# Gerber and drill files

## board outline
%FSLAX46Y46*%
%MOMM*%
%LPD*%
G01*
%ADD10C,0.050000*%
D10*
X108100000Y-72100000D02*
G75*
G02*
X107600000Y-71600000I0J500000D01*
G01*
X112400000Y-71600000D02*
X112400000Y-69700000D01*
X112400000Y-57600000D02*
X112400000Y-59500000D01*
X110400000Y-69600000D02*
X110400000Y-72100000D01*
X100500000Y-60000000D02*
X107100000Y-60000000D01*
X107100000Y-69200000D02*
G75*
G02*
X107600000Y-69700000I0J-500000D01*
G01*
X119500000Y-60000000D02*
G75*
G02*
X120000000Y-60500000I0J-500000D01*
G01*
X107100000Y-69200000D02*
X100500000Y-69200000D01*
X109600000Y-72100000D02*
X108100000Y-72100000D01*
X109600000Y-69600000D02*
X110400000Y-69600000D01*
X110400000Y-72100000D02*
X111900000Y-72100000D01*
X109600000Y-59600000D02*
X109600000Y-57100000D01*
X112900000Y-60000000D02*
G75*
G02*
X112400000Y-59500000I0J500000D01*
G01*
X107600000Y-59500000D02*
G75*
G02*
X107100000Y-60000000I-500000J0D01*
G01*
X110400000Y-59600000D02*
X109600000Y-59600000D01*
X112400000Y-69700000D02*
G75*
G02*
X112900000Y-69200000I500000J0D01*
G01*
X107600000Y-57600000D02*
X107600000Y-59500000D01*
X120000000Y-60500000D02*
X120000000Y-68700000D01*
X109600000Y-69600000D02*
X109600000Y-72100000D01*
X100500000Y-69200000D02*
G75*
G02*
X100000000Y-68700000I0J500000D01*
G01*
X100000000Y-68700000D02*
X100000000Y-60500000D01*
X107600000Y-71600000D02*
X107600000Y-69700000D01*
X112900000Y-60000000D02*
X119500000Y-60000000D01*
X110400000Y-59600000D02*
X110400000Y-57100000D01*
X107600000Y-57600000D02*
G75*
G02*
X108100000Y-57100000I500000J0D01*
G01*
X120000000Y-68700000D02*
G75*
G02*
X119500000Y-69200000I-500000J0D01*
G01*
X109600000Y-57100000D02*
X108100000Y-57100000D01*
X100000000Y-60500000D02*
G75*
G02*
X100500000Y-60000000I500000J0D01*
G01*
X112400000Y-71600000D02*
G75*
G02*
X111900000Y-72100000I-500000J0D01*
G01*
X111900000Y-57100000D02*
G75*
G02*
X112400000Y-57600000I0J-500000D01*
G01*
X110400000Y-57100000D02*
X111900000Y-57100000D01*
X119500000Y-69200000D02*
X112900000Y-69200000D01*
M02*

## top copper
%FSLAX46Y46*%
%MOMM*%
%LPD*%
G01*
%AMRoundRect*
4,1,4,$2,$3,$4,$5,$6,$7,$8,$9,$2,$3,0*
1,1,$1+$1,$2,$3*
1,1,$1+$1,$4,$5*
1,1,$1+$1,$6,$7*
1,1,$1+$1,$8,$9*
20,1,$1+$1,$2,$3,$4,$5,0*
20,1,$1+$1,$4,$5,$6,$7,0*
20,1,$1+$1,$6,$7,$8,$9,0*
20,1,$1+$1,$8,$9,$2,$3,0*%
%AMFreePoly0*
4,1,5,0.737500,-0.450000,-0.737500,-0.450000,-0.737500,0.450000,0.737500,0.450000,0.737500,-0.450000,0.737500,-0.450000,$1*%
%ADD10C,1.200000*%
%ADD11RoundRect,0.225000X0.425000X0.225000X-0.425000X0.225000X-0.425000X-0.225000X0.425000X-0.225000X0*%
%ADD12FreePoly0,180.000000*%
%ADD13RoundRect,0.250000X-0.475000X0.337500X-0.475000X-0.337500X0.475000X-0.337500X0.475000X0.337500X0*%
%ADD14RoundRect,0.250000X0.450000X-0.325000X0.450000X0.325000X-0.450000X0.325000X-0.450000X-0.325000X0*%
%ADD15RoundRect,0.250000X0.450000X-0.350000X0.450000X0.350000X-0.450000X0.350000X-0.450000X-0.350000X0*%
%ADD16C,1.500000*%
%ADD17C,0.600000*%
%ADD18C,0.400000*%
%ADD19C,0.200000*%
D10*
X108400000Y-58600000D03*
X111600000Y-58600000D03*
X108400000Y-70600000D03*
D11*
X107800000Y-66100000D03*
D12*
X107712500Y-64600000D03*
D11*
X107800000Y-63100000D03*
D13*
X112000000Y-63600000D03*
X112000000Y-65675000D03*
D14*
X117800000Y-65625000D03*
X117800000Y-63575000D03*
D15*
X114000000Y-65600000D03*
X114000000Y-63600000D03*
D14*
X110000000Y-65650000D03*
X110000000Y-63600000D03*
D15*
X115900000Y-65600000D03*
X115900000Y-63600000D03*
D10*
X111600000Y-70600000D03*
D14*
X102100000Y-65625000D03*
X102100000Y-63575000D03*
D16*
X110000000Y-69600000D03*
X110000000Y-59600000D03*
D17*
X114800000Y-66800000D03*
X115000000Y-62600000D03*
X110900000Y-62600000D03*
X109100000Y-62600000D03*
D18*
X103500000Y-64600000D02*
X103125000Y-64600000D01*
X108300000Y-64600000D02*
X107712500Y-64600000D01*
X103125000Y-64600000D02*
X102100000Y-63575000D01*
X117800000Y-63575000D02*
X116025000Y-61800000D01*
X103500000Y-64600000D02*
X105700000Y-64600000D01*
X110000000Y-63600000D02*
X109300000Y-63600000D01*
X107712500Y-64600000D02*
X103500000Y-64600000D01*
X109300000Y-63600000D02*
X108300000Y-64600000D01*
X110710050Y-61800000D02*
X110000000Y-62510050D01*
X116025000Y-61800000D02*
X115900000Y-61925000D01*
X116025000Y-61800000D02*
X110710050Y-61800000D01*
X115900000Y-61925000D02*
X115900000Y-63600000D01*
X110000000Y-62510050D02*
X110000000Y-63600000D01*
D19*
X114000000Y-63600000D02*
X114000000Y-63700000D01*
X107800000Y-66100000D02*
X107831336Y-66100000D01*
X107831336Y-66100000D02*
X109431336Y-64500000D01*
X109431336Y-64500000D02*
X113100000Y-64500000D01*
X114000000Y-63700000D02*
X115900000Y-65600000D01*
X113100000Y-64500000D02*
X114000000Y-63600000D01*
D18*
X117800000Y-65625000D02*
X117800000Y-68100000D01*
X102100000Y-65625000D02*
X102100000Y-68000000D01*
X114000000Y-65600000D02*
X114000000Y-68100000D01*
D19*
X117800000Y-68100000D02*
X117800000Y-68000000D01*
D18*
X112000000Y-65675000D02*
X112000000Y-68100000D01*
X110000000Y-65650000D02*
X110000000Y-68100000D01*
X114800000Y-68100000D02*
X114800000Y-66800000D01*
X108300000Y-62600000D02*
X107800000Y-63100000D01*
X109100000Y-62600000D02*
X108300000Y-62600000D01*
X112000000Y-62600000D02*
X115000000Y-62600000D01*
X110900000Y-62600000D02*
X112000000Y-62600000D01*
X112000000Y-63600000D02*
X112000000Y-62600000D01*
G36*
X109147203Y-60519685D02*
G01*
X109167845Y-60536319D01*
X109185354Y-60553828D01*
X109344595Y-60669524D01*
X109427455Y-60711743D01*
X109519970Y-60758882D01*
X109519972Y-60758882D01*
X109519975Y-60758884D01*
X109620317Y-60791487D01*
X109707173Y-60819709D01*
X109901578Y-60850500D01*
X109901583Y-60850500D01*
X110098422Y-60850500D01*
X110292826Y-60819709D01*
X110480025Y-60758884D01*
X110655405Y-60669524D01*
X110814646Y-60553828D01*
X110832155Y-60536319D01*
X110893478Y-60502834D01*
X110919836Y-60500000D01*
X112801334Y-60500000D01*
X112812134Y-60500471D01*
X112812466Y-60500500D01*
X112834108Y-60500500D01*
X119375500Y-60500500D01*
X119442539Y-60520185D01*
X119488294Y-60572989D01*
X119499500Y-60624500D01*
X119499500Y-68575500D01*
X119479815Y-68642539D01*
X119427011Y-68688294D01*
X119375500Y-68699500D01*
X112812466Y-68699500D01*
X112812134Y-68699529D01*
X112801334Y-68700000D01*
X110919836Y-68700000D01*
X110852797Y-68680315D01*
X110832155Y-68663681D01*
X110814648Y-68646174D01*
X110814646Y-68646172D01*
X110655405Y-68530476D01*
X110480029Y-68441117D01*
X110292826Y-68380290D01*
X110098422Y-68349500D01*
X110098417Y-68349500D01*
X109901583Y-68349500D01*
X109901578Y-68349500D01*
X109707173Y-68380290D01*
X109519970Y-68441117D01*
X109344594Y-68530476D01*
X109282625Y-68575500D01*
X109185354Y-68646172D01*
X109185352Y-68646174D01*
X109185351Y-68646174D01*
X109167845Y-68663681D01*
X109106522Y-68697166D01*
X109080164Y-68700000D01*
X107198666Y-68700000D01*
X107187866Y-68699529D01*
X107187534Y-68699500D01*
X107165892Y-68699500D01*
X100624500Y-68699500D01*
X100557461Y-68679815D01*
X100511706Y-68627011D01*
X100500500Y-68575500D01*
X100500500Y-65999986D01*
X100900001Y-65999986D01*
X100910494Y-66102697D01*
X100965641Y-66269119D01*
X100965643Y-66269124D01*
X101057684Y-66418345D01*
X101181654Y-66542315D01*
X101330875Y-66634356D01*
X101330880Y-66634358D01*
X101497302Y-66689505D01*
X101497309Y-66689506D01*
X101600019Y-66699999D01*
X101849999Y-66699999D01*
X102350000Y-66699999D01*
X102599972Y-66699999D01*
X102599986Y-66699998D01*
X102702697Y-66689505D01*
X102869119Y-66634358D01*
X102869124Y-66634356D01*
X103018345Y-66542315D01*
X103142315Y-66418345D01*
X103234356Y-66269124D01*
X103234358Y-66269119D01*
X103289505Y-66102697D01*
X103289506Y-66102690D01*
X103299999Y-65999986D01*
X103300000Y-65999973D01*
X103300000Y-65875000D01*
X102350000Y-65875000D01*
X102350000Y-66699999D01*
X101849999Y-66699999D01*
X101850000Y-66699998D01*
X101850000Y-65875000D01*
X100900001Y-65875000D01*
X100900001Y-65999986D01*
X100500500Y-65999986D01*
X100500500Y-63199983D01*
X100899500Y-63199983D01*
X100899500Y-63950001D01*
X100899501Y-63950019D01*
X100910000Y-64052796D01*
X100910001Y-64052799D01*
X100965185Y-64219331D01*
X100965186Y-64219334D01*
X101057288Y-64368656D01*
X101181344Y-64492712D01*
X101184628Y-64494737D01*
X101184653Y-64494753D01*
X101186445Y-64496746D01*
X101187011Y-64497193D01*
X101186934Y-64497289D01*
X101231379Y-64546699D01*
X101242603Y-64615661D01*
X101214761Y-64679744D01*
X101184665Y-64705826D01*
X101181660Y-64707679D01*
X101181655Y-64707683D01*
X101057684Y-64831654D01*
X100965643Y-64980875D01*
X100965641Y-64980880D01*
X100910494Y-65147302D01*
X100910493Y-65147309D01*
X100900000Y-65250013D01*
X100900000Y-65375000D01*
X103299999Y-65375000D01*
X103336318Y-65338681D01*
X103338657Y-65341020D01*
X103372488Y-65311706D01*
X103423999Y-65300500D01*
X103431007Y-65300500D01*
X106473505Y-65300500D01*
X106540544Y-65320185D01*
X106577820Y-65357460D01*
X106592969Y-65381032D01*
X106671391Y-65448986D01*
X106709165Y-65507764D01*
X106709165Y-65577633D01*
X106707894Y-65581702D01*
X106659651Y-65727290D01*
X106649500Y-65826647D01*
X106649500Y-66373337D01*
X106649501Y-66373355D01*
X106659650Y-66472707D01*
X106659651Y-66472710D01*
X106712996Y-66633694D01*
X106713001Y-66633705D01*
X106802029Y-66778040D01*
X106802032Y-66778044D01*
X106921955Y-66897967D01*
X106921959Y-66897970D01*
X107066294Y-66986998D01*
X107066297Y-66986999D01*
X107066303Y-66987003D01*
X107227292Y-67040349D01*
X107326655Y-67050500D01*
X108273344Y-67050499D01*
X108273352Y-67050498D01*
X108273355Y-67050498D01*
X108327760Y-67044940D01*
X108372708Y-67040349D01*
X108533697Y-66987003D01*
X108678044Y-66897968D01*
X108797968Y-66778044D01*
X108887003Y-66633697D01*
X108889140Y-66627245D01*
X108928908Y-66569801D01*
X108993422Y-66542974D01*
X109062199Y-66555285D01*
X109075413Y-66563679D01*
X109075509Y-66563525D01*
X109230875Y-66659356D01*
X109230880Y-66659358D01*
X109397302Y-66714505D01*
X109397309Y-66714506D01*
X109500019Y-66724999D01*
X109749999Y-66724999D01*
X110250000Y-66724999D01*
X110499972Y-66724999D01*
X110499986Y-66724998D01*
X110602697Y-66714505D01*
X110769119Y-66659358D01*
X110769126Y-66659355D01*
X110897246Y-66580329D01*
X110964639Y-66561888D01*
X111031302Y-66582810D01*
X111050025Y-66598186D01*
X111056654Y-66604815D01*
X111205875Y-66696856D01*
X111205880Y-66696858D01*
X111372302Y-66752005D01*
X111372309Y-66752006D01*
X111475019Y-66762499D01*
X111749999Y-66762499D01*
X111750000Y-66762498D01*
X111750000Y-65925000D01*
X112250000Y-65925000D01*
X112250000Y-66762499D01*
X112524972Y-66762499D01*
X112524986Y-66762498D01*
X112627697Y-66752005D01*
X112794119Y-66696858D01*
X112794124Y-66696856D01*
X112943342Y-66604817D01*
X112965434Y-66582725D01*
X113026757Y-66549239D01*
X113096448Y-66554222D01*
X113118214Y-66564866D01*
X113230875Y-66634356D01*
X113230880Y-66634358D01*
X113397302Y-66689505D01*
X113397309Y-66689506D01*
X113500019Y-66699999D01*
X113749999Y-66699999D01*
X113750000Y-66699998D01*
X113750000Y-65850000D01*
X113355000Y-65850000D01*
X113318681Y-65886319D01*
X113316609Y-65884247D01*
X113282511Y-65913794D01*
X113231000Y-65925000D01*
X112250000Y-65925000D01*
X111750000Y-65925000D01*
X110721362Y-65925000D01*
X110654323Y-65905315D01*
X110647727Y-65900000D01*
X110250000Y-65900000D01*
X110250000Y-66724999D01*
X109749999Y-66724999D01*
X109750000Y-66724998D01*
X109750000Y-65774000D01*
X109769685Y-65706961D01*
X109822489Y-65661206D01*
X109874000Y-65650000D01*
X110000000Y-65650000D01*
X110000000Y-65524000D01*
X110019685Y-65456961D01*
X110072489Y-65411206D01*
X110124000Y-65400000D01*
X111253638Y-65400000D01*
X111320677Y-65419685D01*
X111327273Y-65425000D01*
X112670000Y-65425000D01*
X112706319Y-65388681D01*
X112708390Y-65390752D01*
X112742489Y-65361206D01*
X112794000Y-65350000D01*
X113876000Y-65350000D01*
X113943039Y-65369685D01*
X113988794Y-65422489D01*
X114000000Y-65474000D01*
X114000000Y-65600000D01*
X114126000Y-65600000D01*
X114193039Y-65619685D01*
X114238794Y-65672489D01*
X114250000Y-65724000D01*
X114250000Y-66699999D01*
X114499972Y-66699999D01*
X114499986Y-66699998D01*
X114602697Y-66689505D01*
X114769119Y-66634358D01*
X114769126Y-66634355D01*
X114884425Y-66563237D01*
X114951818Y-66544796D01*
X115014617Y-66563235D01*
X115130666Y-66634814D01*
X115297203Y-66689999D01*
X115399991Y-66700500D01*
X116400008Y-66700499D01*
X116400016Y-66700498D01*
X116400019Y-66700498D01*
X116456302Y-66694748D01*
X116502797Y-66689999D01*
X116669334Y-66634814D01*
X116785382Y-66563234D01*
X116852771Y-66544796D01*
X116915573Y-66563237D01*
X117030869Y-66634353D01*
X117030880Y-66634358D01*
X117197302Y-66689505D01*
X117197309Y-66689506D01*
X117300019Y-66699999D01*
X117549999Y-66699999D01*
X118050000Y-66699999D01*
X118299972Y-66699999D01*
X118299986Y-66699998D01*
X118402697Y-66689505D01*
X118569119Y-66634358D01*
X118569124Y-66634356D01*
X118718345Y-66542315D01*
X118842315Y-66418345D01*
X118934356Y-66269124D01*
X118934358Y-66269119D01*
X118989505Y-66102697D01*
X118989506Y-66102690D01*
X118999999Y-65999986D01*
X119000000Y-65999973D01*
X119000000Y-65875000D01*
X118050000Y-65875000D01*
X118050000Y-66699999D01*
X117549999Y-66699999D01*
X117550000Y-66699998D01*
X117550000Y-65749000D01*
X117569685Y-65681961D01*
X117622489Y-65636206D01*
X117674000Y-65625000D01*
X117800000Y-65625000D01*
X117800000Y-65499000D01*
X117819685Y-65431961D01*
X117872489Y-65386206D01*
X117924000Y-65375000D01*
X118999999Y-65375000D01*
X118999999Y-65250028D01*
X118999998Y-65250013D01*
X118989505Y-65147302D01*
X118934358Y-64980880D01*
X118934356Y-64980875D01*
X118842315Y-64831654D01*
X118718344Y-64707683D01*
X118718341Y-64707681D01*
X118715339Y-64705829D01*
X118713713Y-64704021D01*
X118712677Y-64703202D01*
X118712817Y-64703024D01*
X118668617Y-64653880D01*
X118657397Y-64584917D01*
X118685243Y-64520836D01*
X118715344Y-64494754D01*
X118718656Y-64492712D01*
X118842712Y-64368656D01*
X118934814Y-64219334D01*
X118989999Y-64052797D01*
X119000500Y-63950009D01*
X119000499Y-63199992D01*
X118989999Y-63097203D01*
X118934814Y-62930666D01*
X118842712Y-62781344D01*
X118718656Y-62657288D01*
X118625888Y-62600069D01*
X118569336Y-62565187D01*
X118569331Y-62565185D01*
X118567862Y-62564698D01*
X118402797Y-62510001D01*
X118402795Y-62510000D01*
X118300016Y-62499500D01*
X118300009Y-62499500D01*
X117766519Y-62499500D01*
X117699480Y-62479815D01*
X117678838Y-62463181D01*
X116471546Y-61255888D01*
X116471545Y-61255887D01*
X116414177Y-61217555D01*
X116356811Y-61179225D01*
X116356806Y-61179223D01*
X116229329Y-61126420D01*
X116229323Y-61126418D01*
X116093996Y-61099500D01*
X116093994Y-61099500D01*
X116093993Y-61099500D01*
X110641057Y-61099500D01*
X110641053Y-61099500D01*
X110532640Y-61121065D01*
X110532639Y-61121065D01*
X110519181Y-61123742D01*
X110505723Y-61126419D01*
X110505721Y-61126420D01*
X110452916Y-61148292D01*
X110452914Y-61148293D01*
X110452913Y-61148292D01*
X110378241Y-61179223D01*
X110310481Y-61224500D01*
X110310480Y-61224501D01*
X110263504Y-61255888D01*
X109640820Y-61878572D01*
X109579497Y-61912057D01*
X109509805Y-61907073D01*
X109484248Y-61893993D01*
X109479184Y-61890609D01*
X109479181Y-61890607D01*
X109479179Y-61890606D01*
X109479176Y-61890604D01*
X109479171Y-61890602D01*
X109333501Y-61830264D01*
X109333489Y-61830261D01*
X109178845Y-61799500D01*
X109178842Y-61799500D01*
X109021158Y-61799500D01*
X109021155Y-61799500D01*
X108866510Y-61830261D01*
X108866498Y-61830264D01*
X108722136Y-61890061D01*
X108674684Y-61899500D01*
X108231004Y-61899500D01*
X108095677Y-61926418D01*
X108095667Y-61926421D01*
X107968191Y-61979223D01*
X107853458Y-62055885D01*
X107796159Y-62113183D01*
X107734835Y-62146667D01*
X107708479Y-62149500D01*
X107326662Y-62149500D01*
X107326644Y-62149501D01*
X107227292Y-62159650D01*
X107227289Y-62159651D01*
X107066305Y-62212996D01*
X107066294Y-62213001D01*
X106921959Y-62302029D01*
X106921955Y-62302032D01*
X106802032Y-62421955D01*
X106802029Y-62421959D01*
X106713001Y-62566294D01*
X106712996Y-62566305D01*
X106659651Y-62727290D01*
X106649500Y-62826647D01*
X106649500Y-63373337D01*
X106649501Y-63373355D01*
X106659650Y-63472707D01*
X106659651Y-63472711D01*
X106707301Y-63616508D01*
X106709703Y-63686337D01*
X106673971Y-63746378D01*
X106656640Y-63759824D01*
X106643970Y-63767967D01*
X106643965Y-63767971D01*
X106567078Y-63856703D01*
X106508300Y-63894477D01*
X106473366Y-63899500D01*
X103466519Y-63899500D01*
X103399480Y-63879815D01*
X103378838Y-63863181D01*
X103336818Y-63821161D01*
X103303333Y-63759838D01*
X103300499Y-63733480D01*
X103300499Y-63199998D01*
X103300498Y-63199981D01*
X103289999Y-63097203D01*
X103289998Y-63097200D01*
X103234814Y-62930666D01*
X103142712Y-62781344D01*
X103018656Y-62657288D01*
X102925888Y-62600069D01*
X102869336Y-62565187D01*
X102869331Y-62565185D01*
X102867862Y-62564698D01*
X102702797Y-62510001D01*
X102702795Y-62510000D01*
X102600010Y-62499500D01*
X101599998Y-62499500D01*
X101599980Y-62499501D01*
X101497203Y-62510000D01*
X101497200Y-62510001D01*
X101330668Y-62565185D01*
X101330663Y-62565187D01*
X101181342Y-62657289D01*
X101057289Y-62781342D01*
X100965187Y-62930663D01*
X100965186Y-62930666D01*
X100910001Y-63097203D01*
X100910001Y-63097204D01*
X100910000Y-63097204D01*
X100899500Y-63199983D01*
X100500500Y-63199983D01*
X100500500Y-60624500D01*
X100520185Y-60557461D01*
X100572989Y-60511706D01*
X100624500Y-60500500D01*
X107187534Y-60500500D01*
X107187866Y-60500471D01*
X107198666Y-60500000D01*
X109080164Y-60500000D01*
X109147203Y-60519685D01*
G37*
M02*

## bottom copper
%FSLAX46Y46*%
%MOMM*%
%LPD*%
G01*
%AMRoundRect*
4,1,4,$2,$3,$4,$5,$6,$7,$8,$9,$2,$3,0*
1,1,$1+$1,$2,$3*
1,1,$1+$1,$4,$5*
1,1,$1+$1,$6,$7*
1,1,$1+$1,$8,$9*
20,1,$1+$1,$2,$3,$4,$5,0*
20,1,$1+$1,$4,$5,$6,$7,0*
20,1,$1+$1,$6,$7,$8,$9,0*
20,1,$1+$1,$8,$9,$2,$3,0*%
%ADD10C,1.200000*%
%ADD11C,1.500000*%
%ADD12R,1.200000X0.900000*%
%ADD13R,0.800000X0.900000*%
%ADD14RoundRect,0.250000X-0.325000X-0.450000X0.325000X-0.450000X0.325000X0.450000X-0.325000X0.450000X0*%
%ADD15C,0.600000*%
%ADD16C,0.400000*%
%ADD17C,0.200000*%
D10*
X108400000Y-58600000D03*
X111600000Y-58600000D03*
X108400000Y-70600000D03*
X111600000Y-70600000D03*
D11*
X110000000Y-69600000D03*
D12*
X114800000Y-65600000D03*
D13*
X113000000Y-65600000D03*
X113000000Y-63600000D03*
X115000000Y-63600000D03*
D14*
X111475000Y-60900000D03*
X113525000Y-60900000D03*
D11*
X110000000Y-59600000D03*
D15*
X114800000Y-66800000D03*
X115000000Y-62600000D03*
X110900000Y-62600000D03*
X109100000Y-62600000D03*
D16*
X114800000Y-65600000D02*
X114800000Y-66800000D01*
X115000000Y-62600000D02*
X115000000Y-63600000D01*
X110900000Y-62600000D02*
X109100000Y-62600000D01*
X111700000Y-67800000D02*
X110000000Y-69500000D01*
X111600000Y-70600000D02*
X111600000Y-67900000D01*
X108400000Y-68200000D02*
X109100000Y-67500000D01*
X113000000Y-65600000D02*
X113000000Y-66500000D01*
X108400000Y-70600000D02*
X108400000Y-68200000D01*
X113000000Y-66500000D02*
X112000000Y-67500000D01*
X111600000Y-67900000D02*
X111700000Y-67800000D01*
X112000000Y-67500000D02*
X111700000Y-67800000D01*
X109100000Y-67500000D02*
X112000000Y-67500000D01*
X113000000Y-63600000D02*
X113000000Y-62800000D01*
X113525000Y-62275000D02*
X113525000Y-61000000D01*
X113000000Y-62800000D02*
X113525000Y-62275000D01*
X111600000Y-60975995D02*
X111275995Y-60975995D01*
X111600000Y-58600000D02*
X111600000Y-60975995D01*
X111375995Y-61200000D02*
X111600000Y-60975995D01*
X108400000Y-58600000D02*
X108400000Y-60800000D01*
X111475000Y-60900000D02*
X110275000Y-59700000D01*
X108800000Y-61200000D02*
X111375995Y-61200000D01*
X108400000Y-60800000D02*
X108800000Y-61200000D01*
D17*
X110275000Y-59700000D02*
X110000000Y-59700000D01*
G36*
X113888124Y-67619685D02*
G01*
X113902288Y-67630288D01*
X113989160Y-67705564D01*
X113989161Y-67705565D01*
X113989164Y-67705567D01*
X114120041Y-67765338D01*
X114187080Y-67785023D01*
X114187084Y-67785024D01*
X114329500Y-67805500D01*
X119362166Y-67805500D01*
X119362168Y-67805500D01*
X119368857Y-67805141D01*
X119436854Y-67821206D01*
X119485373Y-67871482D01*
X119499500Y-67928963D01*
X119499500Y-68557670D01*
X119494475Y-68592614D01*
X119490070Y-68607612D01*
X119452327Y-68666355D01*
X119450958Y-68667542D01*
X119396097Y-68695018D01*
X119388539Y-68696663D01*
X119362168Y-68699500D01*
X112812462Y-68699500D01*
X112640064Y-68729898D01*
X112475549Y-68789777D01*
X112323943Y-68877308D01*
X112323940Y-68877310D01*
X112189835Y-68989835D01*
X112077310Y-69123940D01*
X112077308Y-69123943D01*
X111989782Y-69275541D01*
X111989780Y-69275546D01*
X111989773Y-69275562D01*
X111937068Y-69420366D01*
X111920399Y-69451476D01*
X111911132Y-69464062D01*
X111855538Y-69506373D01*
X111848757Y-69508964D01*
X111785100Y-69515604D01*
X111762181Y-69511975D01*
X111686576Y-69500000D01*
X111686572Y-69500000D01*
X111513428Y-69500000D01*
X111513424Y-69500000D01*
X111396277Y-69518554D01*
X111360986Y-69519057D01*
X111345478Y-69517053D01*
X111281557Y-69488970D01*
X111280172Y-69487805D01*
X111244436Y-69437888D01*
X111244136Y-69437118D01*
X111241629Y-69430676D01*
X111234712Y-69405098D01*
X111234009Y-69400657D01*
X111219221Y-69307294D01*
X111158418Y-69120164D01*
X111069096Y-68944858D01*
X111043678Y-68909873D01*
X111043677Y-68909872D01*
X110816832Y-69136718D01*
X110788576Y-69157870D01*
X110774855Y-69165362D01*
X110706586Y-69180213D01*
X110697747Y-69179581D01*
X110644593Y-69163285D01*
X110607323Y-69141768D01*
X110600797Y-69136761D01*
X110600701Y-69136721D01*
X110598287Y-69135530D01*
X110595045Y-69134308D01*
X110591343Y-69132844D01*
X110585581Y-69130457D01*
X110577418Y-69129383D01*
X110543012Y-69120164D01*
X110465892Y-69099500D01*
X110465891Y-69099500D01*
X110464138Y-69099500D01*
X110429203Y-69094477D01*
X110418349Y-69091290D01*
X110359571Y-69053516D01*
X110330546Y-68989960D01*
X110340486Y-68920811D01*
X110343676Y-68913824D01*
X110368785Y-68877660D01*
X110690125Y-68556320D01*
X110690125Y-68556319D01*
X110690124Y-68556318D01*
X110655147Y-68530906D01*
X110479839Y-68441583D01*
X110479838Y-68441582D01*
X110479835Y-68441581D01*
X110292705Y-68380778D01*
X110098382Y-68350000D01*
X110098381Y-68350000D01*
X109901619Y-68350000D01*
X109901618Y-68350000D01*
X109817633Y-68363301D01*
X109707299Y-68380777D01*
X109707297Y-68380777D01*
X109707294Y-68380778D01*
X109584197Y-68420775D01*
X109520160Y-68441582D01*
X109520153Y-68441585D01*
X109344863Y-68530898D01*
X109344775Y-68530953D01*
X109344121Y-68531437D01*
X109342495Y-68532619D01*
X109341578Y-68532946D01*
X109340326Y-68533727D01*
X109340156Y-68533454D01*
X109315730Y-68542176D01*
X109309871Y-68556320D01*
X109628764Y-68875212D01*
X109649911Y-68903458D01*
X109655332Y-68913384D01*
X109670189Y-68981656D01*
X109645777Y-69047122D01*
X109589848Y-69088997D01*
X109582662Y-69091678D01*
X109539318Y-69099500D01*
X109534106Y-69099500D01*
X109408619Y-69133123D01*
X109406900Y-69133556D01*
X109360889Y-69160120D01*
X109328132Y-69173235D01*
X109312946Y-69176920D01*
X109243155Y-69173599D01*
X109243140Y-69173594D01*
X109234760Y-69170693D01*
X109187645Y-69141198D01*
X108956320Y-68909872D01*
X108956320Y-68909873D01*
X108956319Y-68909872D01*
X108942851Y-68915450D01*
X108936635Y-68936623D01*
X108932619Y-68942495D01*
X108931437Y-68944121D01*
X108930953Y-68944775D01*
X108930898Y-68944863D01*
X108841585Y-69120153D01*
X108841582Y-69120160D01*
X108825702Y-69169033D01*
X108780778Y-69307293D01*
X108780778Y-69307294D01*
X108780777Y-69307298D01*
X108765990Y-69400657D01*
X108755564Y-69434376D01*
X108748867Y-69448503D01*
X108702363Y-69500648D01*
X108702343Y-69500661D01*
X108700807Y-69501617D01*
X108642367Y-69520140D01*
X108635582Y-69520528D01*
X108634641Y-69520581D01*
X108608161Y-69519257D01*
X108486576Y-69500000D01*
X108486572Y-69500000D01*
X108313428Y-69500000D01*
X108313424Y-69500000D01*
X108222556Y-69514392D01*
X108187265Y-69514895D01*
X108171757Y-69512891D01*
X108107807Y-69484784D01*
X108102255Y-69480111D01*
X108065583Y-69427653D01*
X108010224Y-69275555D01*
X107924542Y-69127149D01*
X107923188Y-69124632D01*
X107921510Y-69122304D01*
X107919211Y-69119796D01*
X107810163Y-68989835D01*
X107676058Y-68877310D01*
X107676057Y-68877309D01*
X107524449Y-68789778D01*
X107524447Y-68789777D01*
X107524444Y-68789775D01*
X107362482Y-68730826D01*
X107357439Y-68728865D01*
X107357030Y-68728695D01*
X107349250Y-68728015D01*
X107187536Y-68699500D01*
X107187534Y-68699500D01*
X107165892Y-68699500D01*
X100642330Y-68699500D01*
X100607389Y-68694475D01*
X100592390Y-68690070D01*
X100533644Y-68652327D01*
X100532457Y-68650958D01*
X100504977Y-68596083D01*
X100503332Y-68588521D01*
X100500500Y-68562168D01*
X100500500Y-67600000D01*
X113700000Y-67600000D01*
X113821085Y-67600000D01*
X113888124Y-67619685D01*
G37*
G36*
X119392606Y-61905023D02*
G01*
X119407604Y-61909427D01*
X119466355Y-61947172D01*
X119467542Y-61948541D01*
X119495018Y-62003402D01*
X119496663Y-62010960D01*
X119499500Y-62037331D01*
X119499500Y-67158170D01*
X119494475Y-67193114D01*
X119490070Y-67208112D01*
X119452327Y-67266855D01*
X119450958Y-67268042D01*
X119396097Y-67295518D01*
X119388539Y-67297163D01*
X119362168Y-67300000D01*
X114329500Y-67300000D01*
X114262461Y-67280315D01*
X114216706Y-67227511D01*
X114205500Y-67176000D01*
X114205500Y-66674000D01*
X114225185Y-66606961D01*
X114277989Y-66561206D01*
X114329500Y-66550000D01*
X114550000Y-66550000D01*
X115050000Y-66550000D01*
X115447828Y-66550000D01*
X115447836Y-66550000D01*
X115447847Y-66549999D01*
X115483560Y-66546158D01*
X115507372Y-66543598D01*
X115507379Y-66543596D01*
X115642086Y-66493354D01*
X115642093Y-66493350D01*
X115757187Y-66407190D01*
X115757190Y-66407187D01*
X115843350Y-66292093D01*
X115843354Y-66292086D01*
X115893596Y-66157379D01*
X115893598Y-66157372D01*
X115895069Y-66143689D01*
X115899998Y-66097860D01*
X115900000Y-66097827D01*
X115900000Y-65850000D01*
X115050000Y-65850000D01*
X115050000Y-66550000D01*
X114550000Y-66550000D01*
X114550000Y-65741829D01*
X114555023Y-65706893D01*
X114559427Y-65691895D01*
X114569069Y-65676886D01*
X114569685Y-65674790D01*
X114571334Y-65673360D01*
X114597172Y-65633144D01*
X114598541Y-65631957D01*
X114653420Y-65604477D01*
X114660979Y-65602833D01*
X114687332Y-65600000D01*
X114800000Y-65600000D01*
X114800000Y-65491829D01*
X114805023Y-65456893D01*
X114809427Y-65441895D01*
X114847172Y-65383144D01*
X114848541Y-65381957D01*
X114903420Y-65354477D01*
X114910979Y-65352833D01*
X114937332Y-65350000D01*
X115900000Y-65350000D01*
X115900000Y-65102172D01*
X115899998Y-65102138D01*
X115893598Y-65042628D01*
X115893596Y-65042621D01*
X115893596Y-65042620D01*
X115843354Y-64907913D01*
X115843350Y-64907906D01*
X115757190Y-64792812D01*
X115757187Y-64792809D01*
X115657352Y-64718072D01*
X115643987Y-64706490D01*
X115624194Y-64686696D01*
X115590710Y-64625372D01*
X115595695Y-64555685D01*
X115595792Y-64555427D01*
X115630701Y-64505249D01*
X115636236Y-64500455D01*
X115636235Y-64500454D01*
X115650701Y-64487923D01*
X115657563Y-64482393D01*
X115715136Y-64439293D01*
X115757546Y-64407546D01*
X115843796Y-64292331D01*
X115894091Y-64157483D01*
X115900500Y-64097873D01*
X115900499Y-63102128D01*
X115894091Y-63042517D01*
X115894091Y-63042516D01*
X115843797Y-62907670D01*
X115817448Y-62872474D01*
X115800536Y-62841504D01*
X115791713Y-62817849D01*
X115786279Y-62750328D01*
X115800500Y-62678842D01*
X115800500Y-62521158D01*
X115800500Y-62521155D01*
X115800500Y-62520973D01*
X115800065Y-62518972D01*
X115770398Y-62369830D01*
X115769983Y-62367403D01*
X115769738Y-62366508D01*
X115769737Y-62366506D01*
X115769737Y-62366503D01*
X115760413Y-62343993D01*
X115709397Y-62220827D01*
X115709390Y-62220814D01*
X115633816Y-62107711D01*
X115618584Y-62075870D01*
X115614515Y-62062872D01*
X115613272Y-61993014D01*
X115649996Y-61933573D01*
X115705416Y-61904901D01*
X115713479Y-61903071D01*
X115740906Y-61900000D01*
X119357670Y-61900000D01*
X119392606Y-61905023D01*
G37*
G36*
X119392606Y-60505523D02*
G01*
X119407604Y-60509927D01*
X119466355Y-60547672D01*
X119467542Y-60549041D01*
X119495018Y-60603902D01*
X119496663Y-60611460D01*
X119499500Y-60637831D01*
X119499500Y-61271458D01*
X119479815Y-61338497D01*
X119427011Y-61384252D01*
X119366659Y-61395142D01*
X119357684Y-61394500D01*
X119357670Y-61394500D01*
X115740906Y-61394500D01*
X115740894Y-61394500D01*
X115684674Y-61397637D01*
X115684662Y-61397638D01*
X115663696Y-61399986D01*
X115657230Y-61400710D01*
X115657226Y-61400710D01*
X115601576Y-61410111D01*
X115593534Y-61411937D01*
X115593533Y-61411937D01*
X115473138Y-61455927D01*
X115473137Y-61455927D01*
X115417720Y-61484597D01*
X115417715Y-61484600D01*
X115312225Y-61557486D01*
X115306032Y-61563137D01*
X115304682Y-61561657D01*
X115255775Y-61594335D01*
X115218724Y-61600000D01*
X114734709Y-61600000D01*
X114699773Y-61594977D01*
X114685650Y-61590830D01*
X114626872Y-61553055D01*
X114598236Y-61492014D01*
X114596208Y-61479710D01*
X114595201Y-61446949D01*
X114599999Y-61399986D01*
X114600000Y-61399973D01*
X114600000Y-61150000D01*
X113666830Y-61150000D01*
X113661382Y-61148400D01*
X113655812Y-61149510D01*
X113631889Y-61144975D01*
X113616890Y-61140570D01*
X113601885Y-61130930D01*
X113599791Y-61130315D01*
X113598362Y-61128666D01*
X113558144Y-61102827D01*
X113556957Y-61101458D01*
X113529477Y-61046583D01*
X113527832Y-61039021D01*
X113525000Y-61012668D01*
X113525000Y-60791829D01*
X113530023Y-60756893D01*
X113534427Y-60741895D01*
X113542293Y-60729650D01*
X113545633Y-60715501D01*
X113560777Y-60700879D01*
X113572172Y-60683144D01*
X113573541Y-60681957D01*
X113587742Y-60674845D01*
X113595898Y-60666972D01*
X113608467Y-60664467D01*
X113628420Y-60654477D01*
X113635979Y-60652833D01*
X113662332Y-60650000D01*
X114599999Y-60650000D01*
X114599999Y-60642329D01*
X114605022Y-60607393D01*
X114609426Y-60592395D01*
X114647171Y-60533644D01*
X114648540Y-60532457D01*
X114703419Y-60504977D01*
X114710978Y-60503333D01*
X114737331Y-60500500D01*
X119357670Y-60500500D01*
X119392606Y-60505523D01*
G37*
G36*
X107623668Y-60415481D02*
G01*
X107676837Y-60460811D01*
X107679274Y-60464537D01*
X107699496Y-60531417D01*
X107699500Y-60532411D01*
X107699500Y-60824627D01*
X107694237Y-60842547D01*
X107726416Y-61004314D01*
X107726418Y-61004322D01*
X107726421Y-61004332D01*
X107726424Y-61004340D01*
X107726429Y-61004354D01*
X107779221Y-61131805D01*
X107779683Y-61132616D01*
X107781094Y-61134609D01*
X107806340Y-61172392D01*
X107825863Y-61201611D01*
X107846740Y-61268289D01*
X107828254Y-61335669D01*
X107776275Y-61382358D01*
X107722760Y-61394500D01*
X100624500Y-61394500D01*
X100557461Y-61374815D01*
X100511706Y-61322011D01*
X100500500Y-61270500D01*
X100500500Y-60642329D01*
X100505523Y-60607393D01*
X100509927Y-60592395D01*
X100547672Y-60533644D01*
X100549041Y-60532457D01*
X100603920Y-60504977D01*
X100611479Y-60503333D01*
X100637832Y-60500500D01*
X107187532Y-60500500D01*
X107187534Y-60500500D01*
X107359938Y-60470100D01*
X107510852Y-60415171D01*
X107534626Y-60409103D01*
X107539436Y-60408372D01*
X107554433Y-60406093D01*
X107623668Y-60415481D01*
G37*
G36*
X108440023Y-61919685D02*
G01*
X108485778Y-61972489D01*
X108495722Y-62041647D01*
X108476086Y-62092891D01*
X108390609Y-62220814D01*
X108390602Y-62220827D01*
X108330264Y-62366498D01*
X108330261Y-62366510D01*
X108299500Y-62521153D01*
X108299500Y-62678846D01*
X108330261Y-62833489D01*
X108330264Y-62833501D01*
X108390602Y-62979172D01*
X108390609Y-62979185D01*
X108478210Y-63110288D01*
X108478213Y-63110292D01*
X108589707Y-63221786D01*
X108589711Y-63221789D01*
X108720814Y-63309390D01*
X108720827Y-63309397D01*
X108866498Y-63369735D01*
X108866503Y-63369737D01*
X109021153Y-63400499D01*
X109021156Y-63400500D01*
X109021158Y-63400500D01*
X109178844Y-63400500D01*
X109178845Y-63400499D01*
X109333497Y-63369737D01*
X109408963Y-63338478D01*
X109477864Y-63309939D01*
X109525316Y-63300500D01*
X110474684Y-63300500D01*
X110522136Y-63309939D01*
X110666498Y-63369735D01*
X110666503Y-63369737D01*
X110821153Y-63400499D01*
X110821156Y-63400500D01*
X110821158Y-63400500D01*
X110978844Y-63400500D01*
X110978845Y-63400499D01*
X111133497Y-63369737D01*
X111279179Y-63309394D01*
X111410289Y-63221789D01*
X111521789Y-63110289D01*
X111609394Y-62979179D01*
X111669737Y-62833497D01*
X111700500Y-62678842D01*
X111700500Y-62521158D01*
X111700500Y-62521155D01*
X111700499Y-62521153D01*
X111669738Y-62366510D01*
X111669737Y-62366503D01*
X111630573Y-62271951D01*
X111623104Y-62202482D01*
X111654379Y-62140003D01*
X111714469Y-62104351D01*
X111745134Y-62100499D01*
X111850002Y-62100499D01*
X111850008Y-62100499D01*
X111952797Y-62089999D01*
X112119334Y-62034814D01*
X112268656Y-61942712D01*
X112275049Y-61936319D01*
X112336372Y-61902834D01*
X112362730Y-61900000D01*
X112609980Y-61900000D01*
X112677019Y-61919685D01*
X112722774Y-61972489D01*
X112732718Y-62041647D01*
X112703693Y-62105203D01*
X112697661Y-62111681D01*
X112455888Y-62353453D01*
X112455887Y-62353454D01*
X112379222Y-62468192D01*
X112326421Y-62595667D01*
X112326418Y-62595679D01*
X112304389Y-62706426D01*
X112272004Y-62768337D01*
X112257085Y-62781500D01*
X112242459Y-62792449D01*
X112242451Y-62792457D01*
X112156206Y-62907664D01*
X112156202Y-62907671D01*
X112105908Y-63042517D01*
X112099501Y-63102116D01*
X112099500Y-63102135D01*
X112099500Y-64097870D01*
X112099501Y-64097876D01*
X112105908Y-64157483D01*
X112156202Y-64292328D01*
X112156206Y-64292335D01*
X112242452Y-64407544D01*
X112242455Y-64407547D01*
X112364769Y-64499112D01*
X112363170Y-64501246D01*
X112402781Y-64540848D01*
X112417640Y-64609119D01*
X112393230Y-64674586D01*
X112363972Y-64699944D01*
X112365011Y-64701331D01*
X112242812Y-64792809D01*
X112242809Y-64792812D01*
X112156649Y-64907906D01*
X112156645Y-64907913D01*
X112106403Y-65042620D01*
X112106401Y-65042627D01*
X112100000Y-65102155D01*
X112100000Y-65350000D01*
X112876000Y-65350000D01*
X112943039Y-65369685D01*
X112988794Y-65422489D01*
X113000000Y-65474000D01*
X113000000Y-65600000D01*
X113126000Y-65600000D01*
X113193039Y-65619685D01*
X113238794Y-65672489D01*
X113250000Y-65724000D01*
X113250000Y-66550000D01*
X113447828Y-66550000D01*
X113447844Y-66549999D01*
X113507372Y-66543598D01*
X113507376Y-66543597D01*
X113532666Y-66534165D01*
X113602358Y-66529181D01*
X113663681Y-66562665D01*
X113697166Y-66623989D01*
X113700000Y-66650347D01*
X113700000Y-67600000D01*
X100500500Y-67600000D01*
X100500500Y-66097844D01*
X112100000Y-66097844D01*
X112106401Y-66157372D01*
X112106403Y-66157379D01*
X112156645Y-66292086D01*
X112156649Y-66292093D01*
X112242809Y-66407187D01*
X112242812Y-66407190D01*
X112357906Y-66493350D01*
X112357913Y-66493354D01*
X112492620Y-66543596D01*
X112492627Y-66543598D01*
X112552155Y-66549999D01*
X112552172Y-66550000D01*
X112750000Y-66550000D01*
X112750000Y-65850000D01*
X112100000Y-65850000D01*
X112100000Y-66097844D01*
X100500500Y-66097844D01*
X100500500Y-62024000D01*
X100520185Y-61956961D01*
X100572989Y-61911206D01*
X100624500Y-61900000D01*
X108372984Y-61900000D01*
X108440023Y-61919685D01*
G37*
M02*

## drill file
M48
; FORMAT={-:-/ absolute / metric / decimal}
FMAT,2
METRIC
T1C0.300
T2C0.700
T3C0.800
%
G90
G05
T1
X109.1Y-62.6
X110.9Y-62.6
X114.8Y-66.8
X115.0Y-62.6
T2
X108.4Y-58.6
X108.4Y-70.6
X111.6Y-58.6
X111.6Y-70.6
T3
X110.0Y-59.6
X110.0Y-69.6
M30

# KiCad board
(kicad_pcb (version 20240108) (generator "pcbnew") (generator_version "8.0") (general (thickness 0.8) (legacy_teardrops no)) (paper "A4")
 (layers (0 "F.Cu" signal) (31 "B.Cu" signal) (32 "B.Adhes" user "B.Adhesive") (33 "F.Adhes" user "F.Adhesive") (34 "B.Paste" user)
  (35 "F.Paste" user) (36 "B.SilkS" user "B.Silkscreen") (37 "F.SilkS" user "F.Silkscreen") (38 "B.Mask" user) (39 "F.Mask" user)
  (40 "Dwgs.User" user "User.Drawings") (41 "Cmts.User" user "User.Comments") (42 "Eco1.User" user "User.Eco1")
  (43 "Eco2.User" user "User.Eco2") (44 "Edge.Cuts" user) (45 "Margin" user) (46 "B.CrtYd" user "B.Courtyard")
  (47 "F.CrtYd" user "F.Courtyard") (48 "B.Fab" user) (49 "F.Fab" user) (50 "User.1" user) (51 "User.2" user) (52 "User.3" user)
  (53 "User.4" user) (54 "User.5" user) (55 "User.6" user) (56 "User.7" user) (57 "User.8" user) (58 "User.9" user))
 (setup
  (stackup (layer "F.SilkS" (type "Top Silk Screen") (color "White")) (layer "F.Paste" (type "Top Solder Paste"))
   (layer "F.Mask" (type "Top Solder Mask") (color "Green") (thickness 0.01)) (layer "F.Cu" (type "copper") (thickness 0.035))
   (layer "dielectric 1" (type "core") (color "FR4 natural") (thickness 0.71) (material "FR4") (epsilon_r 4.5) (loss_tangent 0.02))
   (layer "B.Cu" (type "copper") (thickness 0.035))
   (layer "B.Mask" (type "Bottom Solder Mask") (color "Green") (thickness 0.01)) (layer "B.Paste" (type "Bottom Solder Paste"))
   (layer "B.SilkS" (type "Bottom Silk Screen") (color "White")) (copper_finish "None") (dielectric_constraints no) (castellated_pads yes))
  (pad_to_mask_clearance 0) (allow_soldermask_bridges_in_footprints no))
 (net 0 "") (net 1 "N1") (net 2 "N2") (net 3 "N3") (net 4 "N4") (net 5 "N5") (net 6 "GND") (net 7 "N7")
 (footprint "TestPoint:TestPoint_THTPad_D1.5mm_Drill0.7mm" (layer "F.Cu") (at 108.4 58.6)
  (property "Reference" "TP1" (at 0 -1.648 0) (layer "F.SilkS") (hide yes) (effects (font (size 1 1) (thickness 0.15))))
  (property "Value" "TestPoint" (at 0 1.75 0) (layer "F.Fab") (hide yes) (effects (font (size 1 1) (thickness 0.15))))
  (pad "1" thru_hole circle (at 0 0) (size 1.2 1.2) (drill 0.7) (layers "*.Cu" "*.Mask") (remove_unused_layers no) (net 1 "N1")))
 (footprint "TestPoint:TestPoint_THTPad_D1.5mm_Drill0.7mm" (layer "F.Cu") (at 111.6 58.6)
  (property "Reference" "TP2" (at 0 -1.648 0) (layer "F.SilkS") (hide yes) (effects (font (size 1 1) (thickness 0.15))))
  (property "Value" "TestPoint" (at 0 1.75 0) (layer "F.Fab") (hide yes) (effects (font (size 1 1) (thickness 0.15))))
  (pad "1" thru_hole circle (at 0 0) (size 1.2 1.2) (drill 0.7) (layers "*.Cu" "*.Mask") (remove_unused_layers no) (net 1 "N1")))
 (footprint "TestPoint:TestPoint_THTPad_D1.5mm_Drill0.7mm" (layer "F.Cu") (at 108.4 70.6)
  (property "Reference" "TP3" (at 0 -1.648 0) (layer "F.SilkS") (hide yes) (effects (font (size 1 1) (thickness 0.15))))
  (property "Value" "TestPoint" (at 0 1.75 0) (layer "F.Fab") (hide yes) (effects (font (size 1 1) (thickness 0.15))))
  (pad "1" thru_hole circle (at 0 0) (size 1.2 1.2) (drill 0.7) (layers "*.Cu" "*.Mask") (remove_unused_layers no) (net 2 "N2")))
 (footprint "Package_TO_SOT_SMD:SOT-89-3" (layer "F.Cu") (at 105.85 64.6 180)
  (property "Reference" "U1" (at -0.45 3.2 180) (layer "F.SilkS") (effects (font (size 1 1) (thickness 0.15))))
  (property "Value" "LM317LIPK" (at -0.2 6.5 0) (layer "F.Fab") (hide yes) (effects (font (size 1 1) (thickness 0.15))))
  (pad "1" smd roundrect (at -1.95 -1.5 180) (size 1.3 0.9) (layers "F.Cu" "F.Paste" "F.Mask") (roundrect_rratio 0.25) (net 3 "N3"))
  (pad "2" smd custom (at -1.8625 0 180) (size 1.475 0.9) (layers "F.Cu" "F.Paste" "F.Mask") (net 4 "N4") (zone_connect 2)
   (thermal_bridge_angle 45) (options (clearance outline) (anchor rect)) (primitives))
  (pad "3" smd roundrect (at -1.95 1.5 180) (size 1.3 0.9) (layers "F.Cu" "F.Paste" "F.Mask") (roundrect_rratio 0.25) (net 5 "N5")))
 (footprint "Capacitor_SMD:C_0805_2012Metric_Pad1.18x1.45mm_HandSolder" (layer "F.Cu") (at 112 64.6375 -90)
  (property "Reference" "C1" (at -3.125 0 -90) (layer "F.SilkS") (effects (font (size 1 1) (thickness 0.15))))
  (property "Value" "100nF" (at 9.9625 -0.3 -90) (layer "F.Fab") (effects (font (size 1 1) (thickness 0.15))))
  (pad "1" smd roundrect (at -1.0375 0 270) (size 1.175 1.45) (layers "F.Cu" "F.Paste" "F.Mask") (roundrect_rratio 0.212766) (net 5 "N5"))
  (pad "2" smd roundrect (at 1.0375 0 270) (size 1.175 1.45) (layers "F.Cu" "F.Paste" "F.Mask") (roundrect_rratio 0.212766) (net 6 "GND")))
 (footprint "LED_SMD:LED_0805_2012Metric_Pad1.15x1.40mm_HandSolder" (layer "F.Cu") (at 117.8 64.6 90)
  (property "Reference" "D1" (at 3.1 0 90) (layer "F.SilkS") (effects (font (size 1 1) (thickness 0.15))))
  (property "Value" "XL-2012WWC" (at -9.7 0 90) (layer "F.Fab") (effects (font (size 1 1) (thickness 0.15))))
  (pad "1" smd roundrect (at -1.025 0 90) (size 1.15 1.4) (layers "F.Cu" "F.Paste" "F.Mask") (roundrect_rratio 0.217391) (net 6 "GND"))
  (pad "2" smd roundrect (at 1.025 0 90) (size 1.15 1.4) (layers "F.Cu" "F.Paste" "F.Mask") (roundrect_rratio 0.217391) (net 4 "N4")))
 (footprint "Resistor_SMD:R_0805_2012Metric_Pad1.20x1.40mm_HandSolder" (layer "F.Cu") (at 114 64.6 90)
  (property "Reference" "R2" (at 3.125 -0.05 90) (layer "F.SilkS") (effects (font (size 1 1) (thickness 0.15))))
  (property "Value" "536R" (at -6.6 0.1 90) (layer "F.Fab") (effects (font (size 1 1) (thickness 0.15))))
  (pad "1" smd roundrect (at -1 0 90) (size 1.2 1.4) (layers "F.Cu" "F.Paste" "F.Mask") (roundrect_rratio 0.208333) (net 6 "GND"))
  (pad "2" smd roundrect (at 1 0 90) (size 1.2 1.4) (layers "F.Cu" "F.Paste" "F.Mask") (roundrect_rratio 0.208333) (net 3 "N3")))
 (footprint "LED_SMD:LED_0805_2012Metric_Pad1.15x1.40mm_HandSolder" (layer "F.Cu") (at 110 64.625 90)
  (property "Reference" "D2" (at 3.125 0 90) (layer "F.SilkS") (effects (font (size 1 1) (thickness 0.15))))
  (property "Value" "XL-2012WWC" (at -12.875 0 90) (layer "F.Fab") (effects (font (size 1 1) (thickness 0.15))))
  (pad "1" smd roundrect (at -1.025 0 90) (size 1.15 1.4) (layers "F.Cu" "F.Paste" "F.Mask") (roundrect_rratio 0.217391) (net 6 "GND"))
  (pad "2" smd roundrect (at 1.025 0 90) (size 1.15 1.4) (layers "F.Cu" "F.Paste" "F.Mask") (roundrect_rratio 0.217391) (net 4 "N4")))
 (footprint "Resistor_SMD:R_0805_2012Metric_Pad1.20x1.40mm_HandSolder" (layer "F.Cu") (at 115.9 64.6 90)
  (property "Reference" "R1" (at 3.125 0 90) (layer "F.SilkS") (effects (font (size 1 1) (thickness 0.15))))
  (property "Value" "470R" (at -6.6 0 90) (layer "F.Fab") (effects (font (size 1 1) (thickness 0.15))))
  (pad "1" smd roundrect (at -1 0 90) (size 1.2 1.4) (layers "F.Cu" "F.Paste" "F.Mask") (roundrect_rratio 0.208333) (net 3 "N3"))
  (pad "2" smd roundrect (at 1 0 90) (size 1.2 1.4) (layers "F.Cu" "F.Paste" "F.Mask") (roundrect_rratio 0.208333) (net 4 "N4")))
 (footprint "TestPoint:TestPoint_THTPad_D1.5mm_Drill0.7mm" (layer "F.Cu") (at 111.6 70.6)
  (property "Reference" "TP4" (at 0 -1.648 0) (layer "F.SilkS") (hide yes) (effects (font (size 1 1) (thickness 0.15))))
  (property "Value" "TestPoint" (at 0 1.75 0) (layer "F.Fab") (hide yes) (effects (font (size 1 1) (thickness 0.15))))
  (pad "1" thru_hole circle (at 0 0) (size 1.2 1.2) (drill 0.7) (layers "*.Cu" "*.Mask") (remove_unused_layers no) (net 2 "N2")))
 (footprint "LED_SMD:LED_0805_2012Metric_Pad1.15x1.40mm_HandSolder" (layer "F.Cu") (at 102.1 64.6 90)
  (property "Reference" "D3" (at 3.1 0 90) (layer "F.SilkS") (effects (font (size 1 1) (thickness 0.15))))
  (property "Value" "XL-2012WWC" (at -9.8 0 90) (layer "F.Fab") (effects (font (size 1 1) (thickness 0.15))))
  (pad "1" smd roundrect (at -1.025 0 90) (size 1.15 1.4) (layers "F.Cu" "F.Paste" "F.Mask") (roundrect_rratio 0.217391) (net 6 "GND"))
  (pad "2" smd roundrect (at 1.025 0 90) (size 1.15 1.4) (layers "F.Cu" "F.Paste" "F.Mask") (roundrect_rratio 0.217391) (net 4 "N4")))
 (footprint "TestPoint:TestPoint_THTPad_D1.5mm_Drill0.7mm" (layer "B.Cu") (at 110 69.6 180)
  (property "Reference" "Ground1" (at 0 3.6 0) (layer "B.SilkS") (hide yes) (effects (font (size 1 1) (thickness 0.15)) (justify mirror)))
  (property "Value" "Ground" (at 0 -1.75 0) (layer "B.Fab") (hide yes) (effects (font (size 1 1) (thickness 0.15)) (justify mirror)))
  (pad "1" thru_hole circle (at 0 0 180) (size 1.5 1.5) (drill 0.8) (layers "*.Cu" "*.Mask") (remove_unused_layers no) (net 2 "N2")))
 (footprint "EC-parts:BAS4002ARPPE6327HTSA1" (layer "B.Cu") (at 114 64.6 180)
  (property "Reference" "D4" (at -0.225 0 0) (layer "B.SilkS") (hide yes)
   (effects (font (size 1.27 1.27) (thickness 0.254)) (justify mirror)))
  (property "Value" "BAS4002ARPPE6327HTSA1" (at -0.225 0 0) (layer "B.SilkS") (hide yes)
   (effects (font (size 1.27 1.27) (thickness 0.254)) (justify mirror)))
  (pad "1" smd rect (at -0.8 -1 90) (size 0.9 1.2) (layers "B.Cu" "B.Paste" "B.Mask") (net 6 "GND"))
  (pad "2" smd rect (at 1 -1 180) (size 0.8 0.9) (layers "B.Cu" "B.Paste" "B.Mask") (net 2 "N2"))
  (pad "3" smd rect (at 1 1 180) (size 0.8 0.9) (layers "B.Cu" "B.Paste" "B.Mask") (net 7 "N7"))
  (pad "4" smd rect (at -1 1 180) (size 0.8 0.9) (layers "B.Cu" "B.Paste" "B.Mask") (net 5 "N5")))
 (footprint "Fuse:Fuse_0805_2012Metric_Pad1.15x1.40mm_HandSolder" (layer "B.Cu") (at 112.5 60.9)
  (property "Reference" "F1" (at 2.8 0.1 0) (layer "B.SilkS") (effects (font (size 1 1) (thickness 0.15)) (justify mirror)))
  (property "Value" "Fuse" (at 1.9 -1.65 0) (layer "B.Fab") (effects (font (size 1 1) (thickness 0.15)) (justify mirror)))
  (pad "1" smd roundrect (at -1.025 0) (size 1.15 1.4) (layers "B.Cu" "B.Paste" "B.Mask") (roundrect_rratio 0.217391) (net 1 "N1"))
  (pad "2" smd roundrect (at 1.025 0) (size 1.15 1.4) (layers "B.Cu" "B.Paste" "B.Mask") (roundrect_rratio 0.217391) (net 7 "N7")))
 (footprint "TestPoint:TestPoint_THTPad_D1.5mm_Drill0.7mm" (layer "B.Cu") (at 110 59.6 180)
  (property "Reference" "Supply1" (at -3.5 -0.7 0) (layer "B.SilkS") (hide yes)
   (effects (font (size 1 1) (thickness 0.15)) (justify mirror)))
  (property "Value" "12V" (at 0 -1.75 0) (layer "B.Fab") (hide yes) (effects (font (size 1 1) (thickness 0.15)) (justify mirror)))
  (pad "1" thru_hole circle (at 0 0 180) (size 1.5 1.5) (drill 0.8) (layers "*.Cu" "*.Mask") (remove_unused_layers no) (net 1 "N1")))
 (gr_arc (start 108.1 72.1) (mid 107.746447 71.953553) (end 107.6 71.6) (stroke (width 0.05) (type default)) (layer "Edge.Cuts"))
 (gr_line (start 112.4 71.6) (end 112.4 69.7) (stroke (width 0.05) (type default)) (layer "Edge.Cuts"))
 (gr_line (start 112.4 57.6) (end 112.4 59.5) (stroke (width 0.05) (type default)) (layer "Edge.Cuts"))
 (gr_line (start 110.4 69.6) (end 110.4 72.1) (stroke (width 0.05) (type default)) (layer "Edge.Cuts"))
 (gr_line (start 100.5 60) (end 107.1 60) (stroke (width 0.05) (type default)) (layer "Edge.Cuts"))
 (gr_arc (start 107.1 69.2) (mid 107.453553 69.346447) (end 107.6 69.7) (stroke (width 0.05) (type default)) (layer "Edge.Cuts"))
 (gr_arc (start 119.5 60) (mid 119.853553 60.146447) (end 120 60.5) (stroke (width 0.05) (type default)) (layer "Edge.Cuts"))
 (gr_line (start 107.1 69.2) (end 100.5 69.2) (stroke (width 0.05) (type default)) (layer "Edge.Cuts"))
 (gr_line (start 109.6 72.1) (end 108.1 72.1) (stroke (width 0.05) (type default)) (layer "Edge.Cuts"))
 (gr_line (start 109.6 69.6) (end 110.4 69.6) (stroke (width 0.05) (type default)) (layer "Edge.Cuts"))
 (gr_line (start 110.4 72.1) (end 111.9 72.1) (stroke (width 0.05) (type default)) (layer "Edge.Cuts"))
 (gr_line (start 109.6 59.6) (end 109.6 57.1) (stroke (width 0.05) (type default)) (layer "Edge.Cuts"))
 (gr_arc (start 112.9 60) (mid 112.546447 59.853553) (end 112.4 59.5) (stroke (width 0.05) (type default)) (layer "Edge.Cuts"))
 (gr_arc (start 107.6 59.5) (mid 107.453553 59.853553) (end 107.1 60) (stroke (width 0.05) (type default)) (layer "Edge.Cuts"))
 (gr_line (start 110.4 59.6) (end 109.6 59.6) (stroke (width 0.05) (type default)) (layer "Edge.Cuts"))
 (gr_arc (start 112.4 69.7) (mid 112.546447 69.346447) (end 112.9 69.2) (stroke (width 0.05) (type default)) (layer "Edge.Cuts"))
 (gr_line (start 107.6 57.6) (end 107.6 59.5) (stroke (width 0.05) (type default)) (layer "Edge.Cuts"))
 (gr_line (start 120 60.5) (end 120 68.7) (stroke (width 0.05) (type default)) (layer "Edge.Cuts"))
 (gr_line (start 109.6 69.6) (end 109.6 72.1) (stroke (width 0.05) (type default)) (layer "Edge.Cuts"))
 (gr_arc (start 100.5 69.2) (mid 100.146447 69.053553) (end 100 68.7) (stroke (width 0.05) (type default)) (layer "Edge.Cuts"))
 (gr_line (start 100 68.7) (end 100 60.5) (stroke (width 0.05) (type default)) (layer "Edge.Cuts"))
 (gr_line (start 107.6 71.6) (end 107.6 69.7) (stroke (width 0.05) (type default)) (layer "Edge.Cuts"))
 (gr_line (start 112.9 60) (end 119.5 60) (stroke (width 0.05) (type default)) (layer "Edge.Cuts"))
 (gr_line (start 110.4 59.6) (end 110.4 57.1) (stroke (width 0.05) (type default)) (layer "Edge.Cuts"))
 (gr_arc (start 107.6 57.6) (mid 107.746447 57.246447) (end 108.1 57.1) (stroke (width 0.05) (type default)) (layer "Edge.Cuts"))
 (gr_arc (start 120 68.7) (mid 119.853553 69.053553) (end 119.5 69.2) (stroke (width 0.05) (type default)) (layer "Edge.Cuts"))
 (gr_line (start 109.6 57.1) (end 108.1 57.1) (stroke (width 0.05) (type default)) (layer "Edge.Cuts"))
 (gr_arc (start 100 60.5) (mid 100.146447 60.146447) (end 100.5 60) (stroke (width 0.05) (type default)) (layer "Edge.Cuts"))
 (gr_arc (start 112.4 71.6) (mid 112.253553 71.953553) (end 111.9 72.1) (stroke (width 0.05) (type default)) (layer "Edge.Cuts"))
 (gr_arc (start 111.9 57.1) (mid 112.253553 57.246447) (end 112.4 57.6) (stroke (width 0.05) (type default)) (layer "Edge.Cuts"))
 (gr_line (start 110.4 57.1) (end 111.9 57.1) (stroke (width 0.05) (type default)) (layer "Edge.Cuts"))
 (gr_line (start 119.5 69.2) (end 112.9 69.2) (stroke (width 0.05) (type default)) (layer "Edge.Cuts"))
 (segment (start 103.5 64.6) (end 103.125 64.6) (width 0.4) (layer "F.Cu") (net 4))
 (segment (start 108.3 64.6) (end 107.7125 64.6) (width 0.4) (layer "F.Cu") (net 4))
 (segment (start 103.125 64.6) (end 102.1 63.575) (width 0.4) (layer "F.Cu") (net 4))
 (segment (start 117.8 63.575) (end 116.025 61.8) (width 0.4) (layer "F.Cu") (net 4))
 (segment (start 103.5 64.6) (end 105.7 64.6) (width 0.4) (layer "F.Cu") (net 4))
 (segment (start 110 63.6) (end 109.3 63.6) (width 0.4) (layer "F.Cu") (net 4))
 (segment (start 107.7125 64.6) (end 103.5 64.6) (width 0.4) (layer "F.Cu") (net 4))
 (segment (start 109.3 63.6) (end 108.3 64.6) (width 0.4) (layer "F.Cu") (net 4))
 (segment (start 110.71005 61.8) (end 110 62.51005) (width 0.4) (layer "F.Cu") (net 4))
 (segment (start 116.025 61.8) (end 115.9 61.925) (width 0.4) (layer "F.Cu") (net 4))
 (segment (start 116.025 61.8) (end 110.71005 61.8) (width 0.4) (layer "F.Cu") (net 4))
 (segment (start 115.9 61.925) (end 115.9 63.6) (width 0.4) (layer "F.Cu") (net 4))
 (segment (start 110 62.51005) (end 110 63.6) (width 0.4) (layer "F.Cu") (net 4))
 (segment (start 114 63.6) (end 114 63.7) (width 0.2) (layer "F.Cu") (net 3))
 (segment (start 107.8 66.1) (end 107.831336 66.1) (width 0.2) (layer "F.Cu") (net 3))
 (segment (start 107.831336 66.1) (end 109.431336 64.5) (width 0.2) (layer "F.Cu") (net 3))
 (segment (start 109.431336 64.5) (end 113.1 64.5) (width 0.2) (layer "F.Cu") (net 3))
 (segment (start 114 63.7) (end 115.9 65.6) (width 0.2) (layer "F.Cu") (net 3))
 (segment (start 113.1 64.5) (end 114 63.6) (width 0.2) (layer "F.Cu") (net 3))
 (segment (start 117.8 65.625) (end 117.8 68.1) (width 0.4) (layer "F.Cu") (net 6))
 (segment (start 102.1 65.625) (end 102.1 68) (width 0.4) (layer "F.Cu") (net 6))
 (segment (start 114 65.6) (end 114 68.1) (width 0.4) (layer "F.Cu") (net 6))
 (segment (start 117.8 68.1) (end 117.8 68) (width 0.2) (layer "F.Cu") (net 6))
 (segment (start 112 65.675) (end 112 68.1) (width 0.4) (layer "F.Cu") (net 6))
 (segment (start 110 65.65) (end 110 68.1) (width 0.4) (layer "F.Cu") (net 6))
 (segment (start 114.8 68.1) (end 114.8 66.8) (width 0.4) (layer "F.Cu") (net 6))
 (via (at 114.8 66.8) (size 0.6) (drill 0.3) (layers "F.Cu" "B.Cu") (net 6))
 (segment (start 114.8 65.6) (end 114.8 66.8) (width 0.4) (layer "B.Cu") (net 6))
 (segment (start 108.3 62.6) (end 107.8 63.1) (width 0.4) (layer "F.Cu") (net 5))
 (segment (start 109.1 62.6) (end 108.3 62.6) (width 0.4) (layer "F.Cu") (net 5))
 (segment (start 112 62.6) (end 115 62.6) (width 0.4) (layer "F.Cu") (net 5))
 (segment (start 110.9 62.6) (end 112 62.6) (width 0.4) (layer "F.Cu") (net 5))
 (segment (start 112 63.6) (end 112 62.6) (width 0.4) (layer "F.Cu") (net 5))
 (via (at 115 62.6) (size 0.6) (drill 0.3) (layers "F.Cu" "B.Cu") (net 5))
 (via (at 110.9 62.6) (size 0.6) (drill 0.3) (layers "F.Cu" "B.Cu") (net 5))
 (via (at 109.1 62.6) (size 0.6) (drill 0.3) (layers "F.Cu" "B.Cu") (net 5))
 (segment (start 115 62.6) (end 115 63.6) (width 0.4) (layer "B.Cu") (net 5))
 (segment (start 110.9 62.6) (end 109.1 62.6) (width 0.4) (layer "B.Cu") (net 5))
 (segment (start 111.7 67.8) (end 110 69.5) (width 0.4) (layer "B.Cu") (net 2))
 (segment (start 111.6 70.6) (end 111.6 67.9) (width 0.4) (layer "B.Cu") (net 2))
 (segment (start 108.4 68.2) (end 109.1 67.5) (width 0.4) (layer "B.Cu") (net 2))
 (segment (start 113 65.6) (end 113 66.5) (width 0.4) (layer "B.Cu") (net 2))
 (segment (start 108.4 70.6) (end 108.4 68.2) (width 0.4) (layer "B.Cu") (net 2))
 (segment (start 113 66.5) (end 112 67.5) (width 0.4) (layer "B.Cu") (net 2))
 (segment (start 111.6 67.9) (end 111.7 67.8) (width 0.4) (layer "B.Cu") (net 2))
 (segment (start 112 67.5) (end 111.7 67.8) (width 0.4) (layer "B.Cu") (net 2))
 (segment (start 109.1 67.5) (end 112 67.5) (width 0.4) (layer "B.Cu") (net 2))
 (segment (start 113 63.6) (end 113 62.8) (width 0.4) (layer "B.Cu") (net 7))
 (segment (start 113.525 62.275) (end 113.525 61) (width 0.4) (layer "B.Cu") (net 7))
 (segment (start 113 62.8) (end 113.525 62.275) (width 0.4) (layer "B.Cu") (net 7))
 (segment (start 111.6 60.975995) (end 111.275995 60.975995) (width 0.4) (layer "B.Cu") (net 1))
 (segment (start 111.6 58.6) (end 111.6 60.975995) (width 0.4) (layer "B.Cu") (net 1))
 (segment (start 111.375995 61.2) (end 111.6 60.975995) (width 0.4) (layer "B.Cu") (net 1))
 (segment (start 108.4 58.6) (end 108.4 60.8) (width 0.4) (layer "B.Cu") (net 1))
 (segment (start 111.475 60.9) (end 110.275 59.7) (width 0.4) (layer "B.Cu") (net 1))
 (segment (start 108.8 61.2) (end 111.375995 61.2) (width 0.4) (layer "B.Cu") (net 1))
 (segment (start 108.4 60.8) (end 108.8 61.2) (width 0.4) (layer "B.Cu") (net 1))
 (segment (start 110.275 59.7) (end 110 59.7) (width 0.2) (layer "B.Cu") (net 1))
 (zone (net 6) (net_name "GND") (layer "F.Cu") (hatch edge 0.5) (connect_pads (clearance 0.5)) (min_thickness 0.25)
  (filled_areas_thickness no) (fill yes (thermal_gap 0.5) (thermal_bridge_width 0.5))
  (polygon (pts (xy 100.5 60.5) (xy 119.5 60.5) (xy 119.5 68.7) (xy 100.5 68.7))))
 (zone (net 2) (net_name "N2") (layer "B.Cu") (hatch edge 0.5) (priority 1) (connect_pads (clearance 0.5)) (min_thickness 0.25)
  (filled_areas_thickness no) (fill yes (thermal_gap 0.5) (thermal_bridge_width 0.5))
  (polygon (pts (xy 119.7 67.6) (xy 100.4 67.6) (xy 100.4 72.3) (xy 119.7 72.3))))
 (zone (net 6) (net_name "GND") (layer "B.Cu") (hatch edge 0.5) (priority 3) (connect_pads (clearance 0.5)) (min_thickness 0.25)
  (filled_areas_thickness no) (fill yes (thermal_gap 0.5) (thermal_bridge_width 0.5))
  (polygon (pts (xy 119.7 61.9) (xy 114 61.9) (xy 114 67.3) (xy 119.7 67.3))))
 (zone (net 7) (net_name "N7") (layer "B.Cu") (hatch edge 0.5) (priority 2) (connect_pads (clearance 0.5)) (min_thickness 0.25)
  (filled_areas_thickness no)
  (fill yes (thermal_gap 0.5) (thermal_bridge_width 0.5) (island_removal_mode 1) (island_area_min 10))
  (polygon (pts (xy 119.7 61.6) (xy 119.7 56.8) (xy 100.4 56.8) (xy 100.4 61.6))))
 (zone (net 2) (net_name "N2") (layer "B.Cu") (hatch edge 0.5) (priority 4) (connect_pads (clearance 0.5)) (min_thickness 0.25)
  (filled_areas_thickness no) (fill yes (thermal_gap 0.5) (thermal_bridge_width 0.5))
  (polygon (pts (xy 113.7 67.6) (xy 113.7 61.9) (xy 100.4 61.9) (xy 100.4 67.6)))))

